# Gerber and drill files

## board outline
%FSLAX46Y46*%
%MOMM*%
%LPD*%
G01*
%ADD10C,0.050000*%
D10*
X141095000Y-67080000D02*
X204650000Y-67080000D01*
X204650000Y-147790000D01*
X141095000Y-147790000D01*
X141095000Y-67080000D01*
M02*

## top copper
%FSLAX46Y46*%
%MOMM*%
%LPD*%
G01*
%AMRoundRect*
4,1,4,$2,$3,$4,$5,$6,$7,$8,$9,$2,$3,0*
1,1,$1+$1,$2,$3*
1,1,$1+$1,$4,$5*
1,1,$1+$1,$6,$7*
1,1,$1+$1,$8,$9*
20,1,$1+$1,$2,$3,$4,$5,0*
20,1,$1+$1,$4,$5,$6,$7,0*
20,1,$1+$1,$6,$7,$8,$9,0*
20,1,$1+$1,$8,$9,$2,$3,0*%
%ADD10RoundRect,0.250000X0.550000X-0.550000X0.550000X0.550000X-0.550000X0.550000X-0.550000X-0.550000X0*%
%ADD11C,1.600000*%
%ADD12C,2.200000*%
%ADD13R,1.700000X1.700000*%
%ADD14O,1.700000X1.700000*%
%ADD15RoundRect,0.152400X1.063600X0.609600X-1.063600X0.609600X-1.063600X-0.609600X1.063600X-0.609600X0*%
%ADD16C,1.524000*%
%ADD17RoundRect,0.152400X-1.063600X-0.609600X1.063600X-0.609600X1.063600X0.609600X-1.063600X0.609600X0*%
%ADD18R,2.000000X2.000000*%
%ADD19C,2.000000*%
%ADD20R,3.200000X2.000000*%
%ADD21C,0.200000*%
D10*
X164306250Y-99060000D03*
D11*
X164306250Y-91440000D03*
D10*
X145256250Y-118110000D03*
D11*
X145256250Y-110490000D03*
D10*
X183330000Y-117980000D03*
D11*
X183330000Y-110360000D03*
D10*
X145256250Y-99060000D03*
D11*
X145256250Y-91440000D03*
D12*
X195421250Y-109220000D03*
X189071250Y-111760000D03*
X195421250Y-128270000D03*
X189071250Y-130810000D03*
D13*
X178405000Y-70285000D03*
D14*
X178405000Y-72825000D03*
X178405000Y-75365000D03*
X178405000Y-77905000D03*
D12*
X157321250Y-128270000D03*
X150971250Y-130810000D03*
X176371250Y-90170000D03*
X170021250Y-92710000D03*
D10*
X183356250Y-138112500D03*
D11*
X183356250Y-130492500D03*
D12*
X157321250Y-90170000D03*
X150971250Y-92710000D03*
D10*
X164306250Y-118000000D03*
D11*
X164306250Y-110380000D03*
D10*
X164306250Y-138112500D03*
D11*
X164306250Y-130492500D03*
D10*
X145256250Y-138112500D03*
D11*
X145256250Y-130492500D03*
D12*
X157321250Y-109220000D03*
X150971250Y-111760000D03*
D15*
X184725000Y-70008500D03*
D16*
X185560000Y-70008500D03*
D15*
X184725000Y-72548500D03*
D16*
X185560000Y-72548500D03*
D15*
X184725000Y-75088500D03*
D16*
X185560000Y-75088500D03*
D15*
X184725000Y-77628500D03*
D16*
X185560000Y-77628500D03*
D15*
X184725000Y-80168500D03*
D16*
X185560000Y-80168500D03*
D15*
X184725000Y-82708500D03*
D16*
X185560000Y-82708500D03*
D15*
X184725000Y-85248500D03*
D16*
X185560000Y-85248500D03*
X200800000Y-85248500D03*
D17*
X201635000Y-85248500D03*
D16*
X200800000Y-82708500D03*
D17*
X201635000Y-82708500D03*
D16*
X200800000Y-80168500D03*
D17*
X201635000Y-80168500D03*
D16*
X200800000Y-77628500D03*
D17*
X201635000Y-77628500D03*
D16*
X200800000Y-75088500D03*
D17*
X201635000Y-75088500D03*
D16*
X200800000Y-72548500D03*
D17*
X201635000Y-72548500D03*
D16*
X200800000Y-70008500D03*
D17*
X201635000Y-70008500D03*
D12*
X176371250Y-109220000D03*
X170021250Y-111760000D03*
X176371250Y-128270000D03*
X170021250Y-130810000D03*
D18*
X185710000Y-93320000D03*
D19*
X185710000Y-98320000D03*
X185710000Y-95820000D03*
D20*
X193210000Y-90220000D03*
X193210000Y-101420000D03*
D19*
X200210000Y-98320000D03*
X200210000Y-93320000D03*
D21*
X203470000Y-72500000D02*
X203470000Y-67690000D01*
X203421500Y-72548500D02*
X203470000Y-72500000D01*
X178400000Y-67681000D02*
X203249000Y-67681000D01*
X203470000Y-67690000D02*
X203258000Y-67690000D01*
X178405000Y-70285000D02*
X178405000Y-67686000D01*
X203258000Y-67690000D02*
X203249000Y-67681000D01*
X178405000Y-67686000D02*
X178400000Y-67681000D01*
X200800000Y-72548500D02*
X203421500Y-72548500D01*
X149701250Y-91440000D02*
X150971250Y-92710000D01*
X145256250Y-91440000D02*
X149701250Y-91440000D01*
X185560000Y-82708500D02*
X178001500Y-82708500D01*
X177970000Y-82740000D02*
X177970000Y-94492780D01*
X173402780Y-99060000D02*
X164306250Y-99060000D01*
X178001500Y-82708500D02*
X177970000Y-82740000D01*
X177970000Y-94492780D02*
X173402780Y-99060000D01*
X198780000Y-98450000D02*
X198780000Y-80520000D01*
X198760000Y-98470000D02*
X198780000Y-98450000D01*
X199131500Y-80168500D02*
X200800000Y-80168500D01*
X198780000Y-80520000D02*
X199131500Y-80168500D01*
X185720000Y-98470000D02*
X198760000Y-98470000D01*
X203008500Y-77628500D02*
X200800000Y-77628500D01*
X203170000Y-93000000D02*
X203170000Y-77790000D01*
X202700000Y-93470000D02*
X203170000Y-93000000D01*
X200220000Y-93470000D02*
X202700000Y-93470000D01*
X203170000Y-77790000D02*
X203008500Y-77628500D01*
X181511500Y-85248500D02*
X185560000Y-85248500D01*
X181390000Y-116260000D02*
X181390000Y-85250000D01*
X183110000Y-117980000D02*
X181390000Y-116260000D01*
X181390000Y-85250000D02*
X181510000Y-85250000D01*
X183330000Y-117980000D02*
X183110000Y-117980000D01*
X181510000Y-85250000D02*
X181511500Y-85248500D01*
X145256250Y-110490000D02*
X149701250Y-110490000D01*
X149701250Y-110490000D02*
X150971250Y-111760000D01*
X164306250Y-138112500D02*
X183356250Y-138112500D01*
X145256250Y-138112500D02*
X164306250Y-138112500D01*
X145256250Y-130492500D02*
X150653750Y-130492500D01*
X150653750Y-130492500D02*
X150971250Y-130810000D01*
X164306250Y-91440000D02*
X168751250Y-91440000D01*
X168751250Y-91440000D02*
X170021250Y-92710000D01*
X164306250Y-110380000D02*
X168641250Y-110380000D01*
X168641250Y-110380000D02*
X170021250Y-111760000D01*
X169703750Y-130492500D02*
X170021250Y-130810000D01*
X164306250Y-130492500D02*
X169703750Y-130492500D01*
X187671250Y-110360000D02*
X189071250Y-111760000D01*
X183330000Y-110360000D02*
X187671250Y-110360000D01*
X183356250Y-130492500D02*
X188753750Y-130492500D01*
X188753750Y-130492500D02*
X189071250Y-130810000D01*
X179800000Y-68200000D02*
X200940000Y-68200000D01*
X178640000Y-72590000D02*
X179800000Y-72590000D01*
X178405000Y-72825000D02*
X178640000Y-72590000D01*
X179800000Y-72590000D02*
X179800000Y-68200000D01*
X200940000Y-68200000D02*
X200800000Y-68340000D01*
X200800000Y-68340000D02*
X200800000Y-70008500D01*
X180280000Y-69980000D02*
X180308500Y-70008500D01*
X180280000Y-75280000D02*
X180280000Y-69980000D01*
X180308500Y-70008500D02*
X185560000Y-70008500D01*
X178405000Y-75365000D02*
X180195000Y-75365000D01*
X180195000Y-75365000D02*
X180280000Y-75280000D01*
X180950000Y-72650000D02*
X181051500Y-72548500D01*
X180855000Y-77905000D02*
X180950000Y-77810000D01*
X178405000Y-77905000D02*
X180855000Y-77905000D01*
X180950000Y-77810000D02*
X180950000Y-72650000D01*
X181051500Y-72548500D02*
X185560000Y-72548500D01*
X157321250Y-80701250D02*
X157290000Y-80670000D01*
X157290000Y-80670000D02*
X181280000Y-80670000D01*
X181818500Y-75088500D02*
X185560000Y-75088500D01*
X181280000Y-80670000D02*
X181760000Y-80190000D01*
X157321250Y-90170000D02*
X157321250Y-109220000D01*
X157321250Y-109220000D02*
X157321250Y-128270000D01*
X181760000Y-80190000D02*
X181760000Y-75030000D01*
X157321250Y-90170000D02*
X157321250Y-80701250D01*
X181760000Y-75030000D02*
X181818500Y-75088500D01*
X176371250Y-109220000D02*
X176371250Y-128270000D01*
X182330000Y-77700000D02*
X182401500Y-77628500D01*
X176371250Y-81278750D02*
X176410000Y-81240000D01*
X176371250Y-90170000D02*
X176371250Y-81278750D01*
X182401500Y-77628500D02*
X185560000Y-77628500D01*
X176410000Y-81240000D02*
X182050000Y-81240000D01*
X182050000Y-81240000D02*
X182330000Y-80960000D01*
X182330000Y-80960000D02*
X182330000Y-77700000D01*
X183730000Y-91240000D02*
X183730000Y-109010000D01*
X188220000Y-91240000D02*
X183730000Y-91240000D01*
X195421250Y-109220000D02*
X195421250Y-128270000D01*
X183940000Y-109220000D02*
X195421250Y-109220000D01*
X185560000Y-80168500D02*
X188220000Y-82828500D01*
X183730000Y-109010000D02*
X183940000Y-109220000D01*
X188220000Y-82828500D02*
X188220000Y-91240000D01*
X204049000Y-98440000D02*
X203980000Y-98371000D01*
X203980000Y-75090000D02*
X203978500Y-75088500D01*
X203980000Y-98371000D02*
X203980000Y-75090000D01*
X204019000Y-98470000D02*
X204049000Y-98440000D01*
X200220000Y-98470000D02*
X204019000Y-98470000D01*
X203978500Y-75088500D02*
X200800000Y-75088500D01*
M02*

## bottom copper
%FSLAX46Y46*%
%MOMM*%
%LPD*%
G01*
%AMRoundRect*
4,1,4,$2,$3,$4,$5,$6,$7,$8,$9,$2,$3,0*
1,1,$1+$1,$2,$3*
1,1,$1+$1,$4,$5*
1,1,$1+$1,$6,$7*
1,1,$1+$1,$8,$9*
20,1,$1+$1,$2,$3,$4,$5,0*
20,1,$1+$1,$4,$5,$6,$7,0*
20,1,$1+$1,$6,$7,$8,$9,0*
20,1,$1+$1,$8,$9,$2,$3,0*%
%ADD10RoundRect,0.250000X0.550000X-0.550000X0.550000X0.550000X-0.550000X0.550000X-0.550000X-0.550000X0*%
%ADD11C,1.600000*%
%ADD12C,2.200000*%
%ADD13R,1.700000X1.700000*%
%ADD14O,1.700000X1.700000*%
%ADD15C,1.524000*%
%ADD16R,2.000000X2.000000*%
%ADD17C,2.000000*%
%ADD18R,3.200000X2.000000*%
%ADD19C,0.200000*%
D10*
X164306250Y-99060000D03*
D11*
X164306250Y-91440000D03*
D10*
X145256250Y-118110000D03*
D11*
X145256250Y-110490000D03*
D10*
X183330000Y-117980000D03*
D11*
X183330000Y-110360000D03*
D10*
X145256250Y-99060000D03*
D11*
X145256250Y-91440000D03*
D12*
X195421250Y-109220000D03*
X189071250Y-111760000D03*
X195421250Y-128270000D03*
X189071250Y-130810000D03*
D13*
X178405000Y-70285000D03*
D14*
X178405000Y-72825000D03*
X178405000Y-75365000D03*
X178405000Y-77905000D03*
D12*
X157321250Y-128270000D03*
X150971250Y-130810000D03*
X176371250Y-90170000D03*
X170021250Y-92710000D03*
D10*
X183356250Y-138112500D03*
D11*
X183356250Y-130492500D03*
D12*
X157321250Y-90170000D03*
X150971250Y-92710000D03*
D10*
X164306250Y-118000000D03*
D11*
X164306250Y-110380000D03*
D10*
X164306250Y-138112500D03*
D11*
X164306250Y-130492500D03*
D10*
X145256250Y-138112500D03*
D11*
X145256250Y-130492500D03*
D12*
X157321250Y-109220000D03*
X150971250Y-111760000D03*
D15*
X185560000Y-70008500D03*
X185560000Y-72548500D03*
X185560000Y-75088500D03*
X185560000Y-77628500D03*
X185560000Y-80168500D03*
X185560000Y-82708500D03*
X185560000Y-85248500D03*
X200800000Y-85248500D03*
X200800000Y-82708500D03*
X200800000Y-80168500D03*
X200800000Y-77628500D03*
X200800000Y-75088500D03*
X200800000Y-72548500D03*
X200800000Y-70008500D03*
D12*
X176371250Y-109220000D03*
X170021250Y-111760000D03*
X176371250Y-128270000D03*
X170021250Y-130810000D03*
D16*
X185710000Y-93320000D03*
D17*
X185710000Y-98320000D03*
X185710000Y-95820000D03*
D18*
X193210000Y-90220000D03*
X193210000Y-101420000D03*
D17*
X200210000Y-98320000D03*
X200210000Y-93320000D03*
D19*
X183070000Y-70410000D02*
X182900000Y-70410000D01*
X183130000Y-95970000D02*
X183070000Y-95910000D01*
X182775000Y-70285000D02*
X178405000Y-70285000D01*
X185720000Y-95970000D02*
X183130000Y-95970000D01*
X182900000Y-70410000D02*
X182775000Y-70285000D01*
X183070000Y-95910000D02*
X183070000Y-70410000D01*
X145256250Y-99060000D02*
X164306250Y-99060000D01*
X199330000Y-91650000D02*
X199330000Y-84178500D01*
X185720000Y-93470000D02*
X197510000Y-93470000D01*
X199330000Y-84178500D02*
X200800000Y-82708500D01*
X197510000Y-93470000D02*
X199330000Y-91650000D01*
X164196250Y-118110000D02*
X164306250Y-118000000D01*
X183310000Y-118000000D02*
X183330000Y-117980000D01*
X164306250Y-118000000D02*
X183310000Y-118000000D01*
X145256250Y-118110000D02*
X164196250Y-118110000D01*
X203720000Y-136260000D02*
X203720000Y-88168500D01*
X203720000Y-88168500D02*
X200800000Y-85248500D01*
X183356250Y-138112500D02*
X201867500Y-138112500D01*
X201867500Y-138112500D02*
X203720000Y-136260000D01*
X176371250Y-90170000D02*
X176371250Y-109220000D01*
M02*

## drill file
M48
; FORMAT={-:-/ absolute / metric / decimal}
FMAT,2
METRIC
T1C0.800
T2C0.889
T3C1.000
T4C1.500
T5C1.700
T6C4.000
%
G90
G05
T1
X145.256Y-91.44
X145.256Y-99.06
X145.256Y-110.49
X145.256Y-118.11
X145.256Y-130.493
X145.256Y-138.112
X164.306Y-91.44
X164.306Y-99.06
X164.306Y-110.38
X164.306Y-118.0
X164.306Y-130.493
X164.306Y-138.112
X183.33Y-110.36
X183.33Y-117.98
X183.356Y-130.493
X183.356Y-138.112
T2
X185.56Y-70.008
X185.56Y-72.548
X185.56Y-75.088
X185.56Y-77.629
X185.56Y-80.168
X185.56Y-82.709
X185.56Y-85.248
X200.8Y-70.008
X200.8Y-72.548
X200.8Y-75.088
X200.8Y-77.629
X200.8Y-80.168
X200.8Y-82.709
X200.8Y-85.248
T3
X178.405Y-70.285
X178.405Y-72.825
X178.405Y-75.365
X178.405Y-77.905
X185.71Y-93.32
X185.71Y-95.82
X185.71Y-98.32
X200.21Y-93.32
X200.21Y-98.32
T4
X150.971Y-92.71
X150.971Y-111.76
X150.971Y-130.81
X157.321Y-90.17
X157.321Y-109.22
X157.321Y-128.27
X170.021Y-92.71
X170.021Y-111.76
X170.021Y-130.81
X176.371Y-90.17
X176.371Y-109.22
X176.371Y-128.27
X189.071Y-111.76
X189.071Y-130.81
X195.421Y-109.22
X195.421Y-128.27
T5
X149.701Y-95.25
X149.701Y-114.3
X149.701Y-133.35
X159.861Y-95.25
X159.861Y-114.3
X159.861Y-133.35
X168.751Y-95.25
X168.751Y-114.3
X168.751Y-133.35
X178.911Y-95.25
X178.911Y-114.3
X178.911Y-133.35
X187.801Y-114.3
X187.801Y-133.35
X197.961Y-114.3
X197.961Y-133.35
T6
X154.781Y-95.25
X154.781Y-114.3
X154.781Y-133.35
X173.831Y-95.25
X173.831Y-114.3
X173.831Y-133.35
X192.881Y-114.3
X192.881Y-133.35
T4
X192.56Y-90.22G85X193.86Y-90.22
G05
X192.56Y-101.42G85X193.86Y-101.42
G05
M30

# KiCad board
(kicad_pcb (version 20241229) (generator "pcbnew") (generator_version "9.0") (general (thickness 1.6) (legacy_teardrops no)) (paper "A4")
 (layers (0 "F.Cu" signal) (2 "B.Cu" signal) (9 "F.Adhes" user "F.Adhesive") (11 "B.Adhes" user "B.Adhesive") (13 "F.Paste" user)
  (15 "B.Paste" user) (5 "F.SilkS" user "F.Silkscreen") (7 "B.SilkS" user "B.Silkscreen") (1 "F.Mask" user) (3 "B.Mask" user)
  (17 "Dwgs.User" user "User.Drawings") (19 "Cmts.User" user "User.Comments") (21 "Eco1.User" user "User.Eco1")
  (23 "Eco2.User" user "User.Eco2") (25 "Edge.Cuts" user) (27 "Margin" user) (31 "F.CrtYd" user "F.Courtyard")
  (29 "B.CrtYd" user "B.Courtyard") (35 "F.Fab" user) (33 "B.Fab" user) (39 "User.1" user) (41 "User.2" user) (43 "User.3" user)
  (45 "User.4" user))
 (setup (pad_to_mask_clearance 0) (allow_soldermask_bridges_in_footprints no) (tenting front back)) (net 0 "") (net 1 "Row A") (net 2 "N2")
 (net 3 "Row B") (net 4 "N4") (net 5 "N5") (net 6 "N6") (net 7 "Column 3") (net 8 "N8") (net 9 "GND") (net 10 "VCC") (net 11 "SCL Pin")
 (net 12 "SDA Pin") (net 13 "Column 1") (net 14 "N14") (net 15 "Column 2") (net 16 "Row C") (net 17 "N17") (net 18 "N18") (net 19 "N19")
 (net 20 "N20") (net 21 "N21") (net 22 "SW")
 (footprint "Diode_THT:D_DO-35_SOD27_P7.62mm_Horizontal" (layer "F.Cu") (at 164.30625 99.06 90)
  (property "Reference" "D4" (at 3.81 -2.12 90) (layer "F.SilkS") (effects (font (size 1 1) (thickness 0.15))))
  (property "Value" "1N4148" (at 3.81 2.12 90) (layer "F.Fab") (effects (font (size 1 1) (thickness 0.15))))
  (pad "1" thru_hole roundrect (at 0 0 90) (size 1.6 1.6) (drill 0.8) (layers "*.Cu" "*.Mask") (remove_unused_layers no)
   (roundrect_rratio 0.15625) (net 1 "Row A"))
  (pad "2" thru_hole circle (at 7.62 0 90) (size 1.6 1.6) (drill 0.8) (layers "*.Cu" "*.Mask") (remove_unused_layers no) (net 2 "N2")))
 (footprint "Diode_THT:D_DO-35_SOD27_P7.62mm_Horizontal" (layer "F.Cu") (at 145.25625 118.11 90)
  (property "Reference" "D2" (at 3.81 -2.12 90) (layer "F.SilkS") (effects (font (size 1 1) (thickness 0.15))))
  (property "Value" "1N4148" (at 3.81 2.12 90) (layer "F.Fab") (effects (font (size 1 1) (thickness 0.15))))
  (pad "1" thru_hole roundrect (at 0 0 90) (size 1.6 1.6) (drill 0.8) (layers "*.Cu" "*.Mask") (remove_unused_layers no)
   (roundrect_rratio 0.15625) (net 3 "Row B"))
  (pad "2" thru_hole circle (at 7.62 0 90) (size 1.6 1.6) (drill 0.8) (layers "*.Cu" "*.Mask") (remove_unused_layers no) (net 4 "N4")))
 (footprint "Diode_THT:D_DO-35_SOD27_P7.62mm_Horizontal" (layer "F.Cu") (at 183.33 117.98 90)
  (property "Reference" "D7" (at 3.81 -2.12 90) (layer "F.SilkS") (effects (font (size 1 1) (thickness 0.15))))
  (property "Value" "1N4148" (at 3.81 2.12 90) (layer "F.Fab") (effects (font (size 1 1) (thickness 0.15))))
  (pad "1" thru_hole roundrect (at 0 0 90) (size 1.6 1.6) (drill 0.8) (layers "*.Cu" "*.Mask") (remove_unused_layers no)
   (roundrect_rratio 0.15625) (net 3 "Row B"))
  (pad "2" thru_hole circle (at 7.62 0 90) (size 1.6 1.6) (drill 0.8) (layers "*.Cu" "*.Mask") (remove_unused_layers no) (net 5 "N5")))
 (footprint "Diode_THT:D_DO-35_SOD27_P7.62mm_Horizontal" (layer "F.Cu") (at 145.25625 99.06 90)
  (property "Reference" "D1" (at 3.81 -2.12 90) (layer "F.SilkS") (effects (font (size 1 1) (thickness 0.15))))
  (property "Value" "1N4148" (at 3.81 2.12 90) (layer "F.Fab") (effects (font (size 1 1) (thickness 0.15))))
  (pad "1" thru_hole roundrect (at 0 0 90) (size 1.6 1.6) (drill 0.8) (layers "*.Cu" "*.Mask") (remove_unused_layers no)
   (roundrect_rratio 0.15625) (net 1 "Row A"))
  (pad "2" thru_hole circle (at 7.62 0 90) (size 1.6 1.6) (drill 0.8) (layers "*.Cu" "*.Mask") (remove_unused_layers no) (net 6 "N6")))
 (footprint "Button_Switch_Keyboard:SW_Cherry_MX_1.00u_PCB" (layer "F.Cu") (at 195.42125 109.22)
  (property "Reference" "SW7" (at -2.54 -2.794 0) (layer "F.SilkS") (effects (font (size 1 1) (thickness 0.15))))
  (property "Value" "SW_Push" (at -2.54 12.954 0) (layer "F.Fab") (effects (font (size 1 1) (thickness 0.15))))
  (pad "" np_thru_hole circle (at -7.62 5.08) (size 1.7 1.7) (drill 1.7) (layers "*.Cu" "*.Mask"))
  (pad "" np_thru_hole circle (at -2.54 5.08) (size 4 4) (drill 4) (layers "*.Cu" "*.Mask"))
  (pad "" np_thru_hole circle (at 2.54 5.08) (size 1.7 1.7) (drill 1.7) (layers "*.Cu" "*.Mask"))
  (pad "1" thru_hole circle (at 0 0) (size 2.2 2.2) (drill 1.5) (layers "*.Cu" "*.Mask") (remove_unused_layers no) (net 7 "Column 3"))
  (pad "2" thru_hole circle (at -6.35 2.54) (size 2.2 2.2) (drill 1.5) (layers "*.Cu" "*.Mask") (remove_unused_layers no) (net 5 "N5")))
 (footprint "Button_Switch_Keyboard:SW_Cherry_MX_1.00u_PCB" (layer "F.Cu") (at 195.42125 128.27)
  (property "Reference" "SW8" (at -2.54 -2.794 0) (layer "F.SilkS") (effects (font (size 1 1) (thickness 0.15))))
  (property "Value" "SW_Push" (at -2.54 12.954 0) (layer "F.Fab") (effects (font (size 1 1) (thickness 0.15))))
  (pad "" np_thru_hole circle (at -7.62 5.08) (size 1.7 1.7) (drill 1.7) (layers "*.Cu" "*.Mask"))
  (pad "" np_thru_hole circle (at -2.54 5.08) (size 4 4) (drill 4) (layers "*.Cu" "*.Mask"))
  (pad "" np_thru_hole circle (at 2.54 5.08) (size 1.7 1.7) (drill 1.7) (layers "*.Cu" "*.Mask"))
  (pad "1" thru_hole circle (at 0 0) (size 2.2 2.2) (drill 1.5) (layers "*.Cu" "*.Mask") (remove_unused_layers no) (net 7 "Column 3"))
  (pad "2" thru_hole circle (at -6.35 2.54) (size 2.2 2.2) (drill 1.5) (layers "*.Cu" "*.Mask") (remove_unused_layers no) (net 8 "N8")))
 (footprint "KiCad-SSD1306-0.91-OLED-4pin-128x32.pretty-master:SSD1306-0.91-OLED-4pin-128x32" (layer "F.Cu") (at 141.905 68.095)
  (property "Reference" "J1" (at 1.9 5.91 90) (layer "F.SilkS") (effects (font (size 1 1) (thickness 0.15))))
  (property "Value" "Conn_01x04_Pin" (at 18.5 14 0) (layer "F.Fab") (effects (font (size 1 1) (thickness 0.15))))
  (pad "1" thru_hole rect (at 36.5 2.19) (size 1.7 1.7) (drill 1) (layers "*.Cu" "*.Mask") (remove_unused_layers no) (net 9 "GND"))
  (pad "2" thru_hole oval (at 36.5 4.73) (size 1.7 1.7) (drill 1) (layers "*.Cu" "*.Mask") (remove_unused_layers no) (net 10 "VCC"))
  (pad "3" thru_hole oval (at 36.5 7.27) (size 1.7 1.7) (drill 1) (layers "*.Cu" "*.Mask") (remove_unused_layers no) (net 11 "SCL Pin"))
  (pad "4" thru_hole oval (at 36.5 9.81) (size 1.7 1.7) (drill 1) (layers "*.Cu" "*.Mask") (remove_unused_layers no) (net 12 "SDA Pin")))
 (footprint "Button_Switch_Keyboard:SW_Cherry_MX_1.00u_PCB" (layer "F.Cu") (at 157.32125 128.27)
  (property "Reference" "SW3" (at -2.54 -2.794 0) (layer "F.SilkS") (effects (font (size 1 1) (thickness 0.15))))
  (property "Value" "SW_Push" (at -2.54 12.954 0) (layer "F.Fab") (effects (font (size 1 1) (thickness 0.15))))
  (pad "" np_thru_hole circle (at -7.62 5.08) (size 1.7 1.7) (drill 1.7) (layers "*.Cu" "*.Mask"))
  (pad "" np_thru_hole circle (at -2.54 5.08) (size 4 4) (drill 4) (layers "*.Cu" "*.Mask"))
  (pad "" np_thru_hole circle (at 2.54 5.08) (size 1.7 1.7) (drill 1.7) (layers "*.Cu" "*.Mask"))
  (pad "1" thru_hole circle (at 0 0) (size 2.2 2.2) (drill 1.5) (layers "*.Cu" "*.Mask") (remove_unused_layers no) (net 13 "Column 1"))
  (pad "2" thru_hole circle (at -6.35 2.54) (size 2.2 2.2) (drill 1.5) (layers "*.Cu" "*.Mask") (remove_unused_layers no) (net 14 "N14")))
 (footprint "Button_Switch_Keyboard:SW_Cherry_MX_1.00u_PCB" (layer "F.Cu") (at 176.37125 90.17)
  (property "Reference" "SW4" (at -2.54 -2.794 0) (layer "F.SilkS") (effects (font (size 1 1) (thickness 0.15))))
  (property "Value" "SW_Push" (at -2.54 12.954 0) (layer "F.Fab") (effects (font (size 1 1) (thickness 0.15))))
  (pad "" np_thru_hole circle (at -7.62 5.08) (size 1.7 1.7) (drill 1.7) (layers "*.Cu" "*.Mask"))
  (pad "" np_thru_hole circle (at -2.54 5.08) (size 4 4) (drill 4) (layers "*.Cu" "*.Mask"))
  (pad "" np_thru_hole circle (at 2.54 5.08) (size 1.7 1.7) (drill 1.7) (layers "*.Cu" "*.Mask"))
  (pad "1" thru_hole circle (at 0 0) (size 2.2 2.2) (drill 1.5) (layers "*.Cu" "*.Mask") (remove_unused_layers no) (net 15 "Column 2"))
  (pad "2" thru_hole circle (at -6.35 2.54) (size 2.2 2.2) (drill 1.5) (layers "*.Cu" "*.Mask") (remove_unused_layers no) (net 2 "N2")))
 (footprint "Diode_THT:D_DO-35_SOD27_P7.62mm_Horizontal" (layer "F.Cu") (at 183.35625 138.1125 90)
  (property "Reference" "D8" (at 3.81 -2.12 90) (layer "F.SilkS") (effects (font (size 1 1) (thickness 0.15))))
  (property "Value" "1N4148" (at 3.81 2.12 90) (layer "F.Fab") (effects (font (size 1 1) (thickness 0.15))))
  (pad "1" thru_hole roundrect (at 0 0 90) (size 1.6 1.6) (drill 0.8) (layers "*.Cu" "*.Mask") (remove_unused_layers no)
   (roundrect_rratio 0.15625) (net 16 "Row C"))
  (pad "2" thru_hole circle (at 7.62 0 90) (size 1.6 1.6) (drill 0.8) (layers "*.Cu" "*.Mask") (remove_unused_layers no) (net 8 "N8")))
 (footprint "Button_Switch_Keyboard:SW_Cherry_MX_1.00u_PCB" (layer "F.Cu") (at 157.32125 90.17)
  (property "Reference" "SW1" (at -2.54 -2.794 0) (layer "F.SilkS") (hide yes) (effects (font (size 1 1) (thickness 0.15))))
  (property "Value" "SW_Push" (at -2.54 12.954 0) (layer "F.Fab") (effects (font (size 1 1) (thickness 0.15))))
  (pad "" np_thru_hole circle (at -7.62 5.08) (size 1.7 1.7) (drill 1.7) (layers "*.Cu" "*.Mask"))
  (pad "" np_thru_hole circle (at -2.54 5.08) (size 4 4) (drill 4) (layers "*.Cu" "*.Mask"))
  (pad "" np_thru_hole circle (at 2.54 5.08) (size 1.7 1.7) (drill 1.7) (layers "*.Cu" "*.Mask"))
  (pad "1" thru_hole circle (at 0 0) (size 2.2 2.2) (drill 1.5) (layers "*.Cu" "*.Mask") (remove_unused_layers no) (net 13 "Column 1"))
  (pad "2" thru_hole circle (at -6.35 2.54) (size 2.2 2.2) (drill 1.5) (layers "*.Cu" "*.Mask") (remove_unused_layers no) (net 6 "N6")))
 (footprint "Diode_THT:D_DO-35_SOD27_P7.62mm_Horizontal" (layer "F.Cu") (at 164.30625 118 90)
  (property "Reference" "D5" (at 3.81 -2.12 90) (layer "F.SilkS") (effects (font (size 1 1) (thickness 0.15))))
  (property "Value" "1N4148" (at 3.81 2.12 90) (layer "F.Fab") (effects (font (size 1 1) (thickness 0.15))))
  (pad "1" thru_hole roundrect (at 0 0 90) (size 1.6 1.6) (drill 0.8) (layers "*.Cu" "*.Mask") (remove_unused_layers no)
   (roundrect_rratio 0.15625) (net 3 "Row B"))
  (pad "2" thru_hole circle (at 7.62 0 90) (size 1.6 1.6) (drill 0.8) (layers "*.Cu" "*.Mask") (remove_unused_layers no) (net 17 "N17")))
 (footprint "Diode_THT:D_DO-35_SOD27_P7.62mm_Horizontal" (layer "F.Cu") (at 164.30625 138.1125 90)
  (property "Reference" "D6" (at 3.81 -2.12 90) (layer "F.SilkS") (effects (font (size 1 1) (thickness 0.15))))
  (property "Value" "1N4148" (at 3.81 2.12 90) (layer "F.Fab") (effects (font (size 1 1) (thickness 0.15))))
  (pad "1" thru_hole roundrect (at 0 0 90) (size 1.6 1.6) (drill 0.8) (layers "*.Cu" "*.Mask") (remove_unused_layers no)
   (roundrect_rratio 0.15625) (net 16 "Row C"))
  (pad "2" thru_hole circle (at 7.62 0 90) (size 1.6 1.6) (drill 0.8) (layers "*.Cu" "*.Mask") (remove_unused_layers no) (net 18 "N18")))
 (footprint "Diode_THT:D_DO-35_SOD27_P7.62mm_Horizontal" (layer "F.Cu") (at 145.25625 138.1125 90)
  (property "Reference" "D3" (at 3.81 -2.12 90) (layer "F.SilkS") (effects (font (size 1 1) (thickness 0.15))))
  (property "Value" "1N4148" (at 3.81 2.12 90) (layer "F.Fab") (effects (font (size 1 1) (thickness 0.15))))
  (pad "1" thru_hole roundrect (at 0 0 90) (size 1.6 1.6) (drill 0.8) (layers "*.Cu" "*.Mask") (remove_unused_layers no)
   (roundrect_rratio 0.15625) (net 16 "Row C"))
  (pad "2" thru_hole circle (at 7.62 0 90) (size 1.6 1.6) (drill 0.8) (layers "*.Cu" "*.Mask") (remove_unused_layers no) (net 14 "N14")))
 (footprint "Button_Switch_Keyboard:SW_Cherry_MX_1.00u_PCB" (layer "F.Cu") (at 157.32125 109.22)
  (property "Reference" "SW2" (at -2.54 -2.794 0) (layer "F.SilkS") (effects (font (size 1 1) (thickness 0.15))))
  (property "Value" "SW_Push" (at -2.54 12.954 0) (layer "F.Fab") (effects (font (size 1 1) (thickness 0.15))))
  (pad "" np_thru_hole circle (at -7.62 5.08) (size 1.7 1.7) (drill 1.7) (layers "*.Cu" "*.Mask"))
  (pad "" np_thru_hole circle (at -2.54 5.08) (size 4 4) (drill 4) (layers "*.Cu" "*.Mask"))
  (pad "" np_thru_hole circle (at 2.54 5.08) (size 1.7 1.7) (drill 1.7) (layers "*.Cu" "*.Mask"))
  (pad "1" thru_hole circle (at 0 0) (size 2.2 2.2) (drill 1.5) (layers "*.Cu" "*.Mask") (remove_unused_layers no) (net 13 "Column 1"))
  (pad "2" thru_hole circle (at -6.35 2.54) (size 2.2 2.2) (drill 1.5) (layers "*.Cu" "*.Mask") (remove_unused_layers no) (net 4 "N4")))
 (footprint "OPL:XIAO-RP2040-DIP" (layer "F.Cu") (at 193.18 77.6285)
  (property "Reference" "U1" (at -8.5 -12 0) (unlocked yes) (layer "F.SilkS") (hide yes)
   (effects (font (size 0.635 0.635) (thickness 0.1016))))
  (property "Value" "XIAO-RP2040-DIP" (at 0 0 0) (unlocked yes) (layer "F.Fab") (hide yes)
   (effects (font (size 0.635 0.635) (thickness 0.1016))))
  (pad "1" smd roundrect (at -8.455 -7.62 180) (size 2.432 1.524) (layers "F.Cu" "F.Mask") (roundrect_rratio 0.1) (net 11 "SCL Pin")
   (thermal_bridge_angle 45))
  (pad "1" thru_hole circle (at -7.62 -7.62 180) (size 1.524 1.524) (drill 0.889) (layers "*.Cu" "*.Mask") (remove_unused_layers no)
   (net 11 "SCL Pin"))
  (pad "2" smd roundrect (at -8.455 -5.08 180) (size 2.432 1.524) (layers "F.Cu" "F.Mask") (roundrect_rratio 0.1) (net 12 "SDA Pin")
   (thermal_bridge_angle 45))
  (pad "2" thru_hole circle (at -7.62 -5.08 180) (size 1.524 1.524) (drill 0.889) (layers "*.Cu" "*.Mask") (remove_unused_layers no)
   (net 12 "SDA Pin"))
  (pad "3" smd roundrect (at -8.455 -2.54 180) (size 2.432 1.524) (layers "F.Cu" "F.Mask") (roundrect_rratio 0.1) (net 13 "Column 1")
   (thermal_bridge_angle 45))
  (pad "3" thru_hole circle (at -7.62 -2.54 180) (size 1.524 1.524) (drill 0.889) (layers "*.Cu" "*.Mask") (remove_unused_layers no)
   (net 13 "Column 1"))
  (pad "4" smd roundrect (at -8.455 0 180) (size 2.432 1.524) (layers "F.Cu" "F.Mask") (roundrect_rratio 0.1) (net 15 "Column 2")
   (thermal_bridge_angle 45))
  (pad "4" thru_hole circle (at -7.62 0 180) (size 1.524 1.524) (drill 0.889) (layers "*.Cu" "*.Mask") (remove_unused_layers no)
   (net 15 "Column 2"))
  (pad "5" smd roundrect (at -8.455 2.54 180) (size 2.432 1.524) (layers "F.Cu" "F.Mask") (roundrect_rratio 0.1) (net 7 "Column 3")
   (thermal_bridge_angle 45))
  (pad "5" thru_hole circle (at -7.62 2.54 180) (size 1.524 1.524) (drill 0.889) (layers "*.Cu" "*.Mask") (remove_unused_layers no)
   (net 7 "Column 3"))
  (pad "6" smd roundrect (at -8.455 5.08 180) (size 2.432 1.524) (layers "F.Cu" "F.Mask") (roundrect_rratio 0.1) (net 1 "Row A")
   (thermal_bridge_angle 45))
  (pad "6" thru_hole circle (at -7.62 5.08 180) (size 1.524 1.524) (drill 0.889) (layers "*.Cu" "*.Mask") (remove_unused_layers no)
   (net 1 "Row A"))
  (pad "7" smd roundrect (at -8.455 7.62 180) (size 2.432 1.524) (layers "F.Cu" "F.Mask") (roundrect_rratio 0.1) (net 3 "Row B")
   (thermal_bridge_angle 45))
  (pad "7" thru_hole circle (at -7.62 7.62 180) (size 1.524 1.524) (drill 0.889) (layers "*.Cu" "*.Mask") (remove_unused_layers no)
   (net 3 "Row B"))
  (pad "8" thru_hole circle (at 7.62 7.62) (size 1.524 1.524) (drill 0.889) (layers "*.Cu" "*.Mask") (remove_unused_layers no)
   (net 16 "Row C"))
  (pad "8" smd roundrect (at 8.455 7.62) (size 2.432 1.524) (layers "F.Cu" "F.Mask") (roundrect_rratio 0.1) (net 16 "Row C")
   (thermal_bridge_angle 45))
  (pad "9" thru_hole circle (at 7.62 5.08) (size 1.524 1.524) (drill 0.889) (layers "*.Cu" "*.Mask") (remove_unused_layers no)
   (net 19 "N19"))
  (pad "9" smd roundrect (at 8.455 5.08) (size 2.432 1.524) (layers "F.Cu" "F.Mask") (roundrect_rratio 0.1) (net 19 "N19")
   (thermal_bridge_angle 45))
  (pad "10" thru_hole circle (at 7.62 2.54) (size 1.524 1.524) (drill 0.889) (layers "*.Cu" "*.Mask") (remove_unused_layers no)
   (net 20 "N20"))
  (pad "10" smd roundrect (at 8.455 2.54) (size 2.432 1.524) (layers "F.Cu" "F.Mask") (roundrect_rratio 0.1) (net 20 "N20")
   (thermal_bridge_angle 45))
  (pad "11" thru_hole circle (at 7.62 0) (size 1.524 1.524) (drill 0.889) (layers "*.Cu" "*.Mask") (remove_unused_layers no) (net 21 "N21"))
  (pad "11" smd roundrect (at 8.455 0) (size 2.432 1.524) (layers "F.Cu" "F.Mask") (roundrect_rratio 0.1) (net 21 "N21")
   (thermal_bridge_angle 45))
  (pad "12" thru_hole circle (at 7.62 -2.54) (size 1.524 1.524) (drill 0.889) (layers "*.Cu" "*.Mask") (remove_unused_layers no)
   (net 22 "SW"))
  (pad "12" smd roundrect (at 8.455 -2.54) (size 2.432 1.524) (layers "F.Cu" "F.Mask") (roundrect_rratio 0.1) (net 22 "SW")
   (thermal_bridge_angle 45))
  (pad "13" thru_hole circle (at 7.62 -5.08) (size 1.524 1.524) (drill 0.889) (layers "*.Cu" "*.Mask") (remove_unused_layers no)
   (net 9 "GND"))
  (pad "13" smd roundrect (at 8.455 -5.08) (size 2.432 1.524) (layers "F.Cu" "F.Mask") (roundrect_rratio 0.1) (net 9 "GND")
   (thermal_bridge_angle 45))
  (pad "14" thru_hole circle (at 7.62 -7.62) (size 1.524 1.524) (drill 0.889) (layers "*.Cu" "*.Mask") (remove_unused_layers no)
   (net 10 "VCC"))
  (pad "14" smd roundrect (at 8.455 -7.62) (size 2.432 1.524) (layers "F.Cu" "F.Mask") (roundrect_rratio 0.1) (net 10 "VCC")
   (thermal_bridge_angle 45)))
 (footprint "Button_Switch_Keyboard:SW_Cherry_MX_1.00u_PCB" (layer "F.Cu") (at 176.37125 109.22)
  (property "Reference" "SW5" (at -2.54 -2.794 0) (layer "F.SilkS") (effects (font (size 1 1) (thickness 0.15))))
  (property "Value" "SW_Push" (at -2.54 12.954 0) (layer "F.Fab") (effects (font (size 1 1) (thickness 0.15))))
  (pad "" np_thru_hole circle (at -7.62 5.08) (size 1.7 1.7) (drill 1.7) (layers "*.Cu" "*.Mask"))
  (pad "" np_thru_hole circle (at -2.54 5.08) (size 4 4) (drill 4) (layers "*.Cu" "*.Mask"))
  (pad "" np_thru_hole circle (at 2.54 5.08) (size 1.7 1.7) (drill 1.7) (layers "*.Cu" "*.Mask"))
  (pad "1" thru_hole circle (at 0 0) (size 2.2 2.2) (drill 1.5) (layers "*.Cu" "*.Mask") (remove_unused_layers no) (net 15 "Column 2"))
  (pad "2" thru_hole circle (at -6.35 2.54) (size 2.2 2.2) (drill 1.5) (layers "*.Cu" "*.Mask") (remove_unused_layers no) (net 17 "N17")))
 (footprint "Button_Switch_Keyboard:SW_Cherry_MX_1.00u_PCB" (layer "F.Cu") (at 176.37125 128.27)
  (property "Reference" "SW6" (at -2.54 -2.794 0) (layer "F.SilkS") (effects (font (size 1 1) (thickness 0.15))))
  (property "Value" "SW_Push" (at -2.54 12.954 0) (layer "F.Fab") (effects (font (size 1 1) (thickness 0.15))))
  (pad "" np_thru_hole circle (at -7.62 5.08) (size 1.7 1.7) (drill 1.7) (layers "*.Cu" "*.Mask"))
  (pad "" np_thru_hole circle (at -2.54 5.08) (size 4 4) (drill 4) (layers "*.Cu" "*.Mask"))
  (pad "" np_thru_hole circle (at 2.54 5.08) (size 1.7 1.7) (drill 1.7) (layers "*.Cu" "*.Mask"))
  (pad "1" thru_hole circle (at 0 0) (size 2.2 2.2) (drill 1.5) (layers "*.Cu" "*.Mask") (remove_unused_layers no) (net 15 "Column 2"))
  (pad "2" thru_hole circle (at -6.35 2.54) (size 2.2 2.2) (drill 1.5) (layers "*.Cu" "*.Mask") (remove_unused_layers no) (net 18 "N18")))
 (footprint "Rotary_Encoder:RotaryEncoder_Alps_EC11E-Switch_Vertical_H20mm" (layer "F.Cu") (at 185.71 93.32)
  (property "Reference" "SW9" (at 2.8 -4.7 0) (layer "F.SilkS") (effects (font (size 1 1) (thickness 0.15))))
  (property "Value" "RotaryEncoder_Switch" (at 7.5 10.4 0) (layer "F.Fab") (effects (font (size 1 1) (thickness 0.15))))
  (pad "A" thru_hole rect (at 0 0) (size 2 2) (drill 1) (layers "*.Cu" "*.Mask") (remove_unused_layers no) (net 19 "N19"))
  (pad "B" thru_hole circle (at 0 5) (size 2 2) (drill 1) (layers "*.Cu" "*.Mask") (remove_unused_layers no) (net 20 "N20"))
  (pad "C" thru_hole circle (at 0 2.5) (size 2 2) (drill 1) (layers "*.Cu" "*.Mask") (remove_unused_layers no) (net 9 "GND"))
  (pad "MP" thru_hole rect (at 7.5 -3.1) (size 3.2 2) (drill oval 2.8 1.5) (layers "*.Cu" "*.Mask") (remove_unused_layers no))
  (pad "MP" thru_hole rect (at 7.5 8.1) (size 3.2 2) (drill oval 2.8 1.5) (layers "*.Cu" "*.Mask") (remove_unused_layers no))
  (pad "S1" thru_hole circle (at 14.5 5) (size 2 2) (drill 1) (layers "*.Cu" "*.Mask") (remove_unused_layers no) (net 22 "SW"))
  (pad "S2" thru_hole circle (at 14.5 0) (size 2 2) (drill 1) (layers "*.Cu" "*.Mask") (remove_unused_layers no) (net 21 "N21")))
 (gr_rect (start 141.095 67.08) (end 204.65 147.79) (stroke (width 0.05) (type default)) (fill no) (layer "Edge.Cuts"))
 (segment (start 203.47 72.5) (end 203.47 67.69) (width 0.2) (layer "F.Cu") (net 9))
 (segment (start 203.4215 72.5485) (end 203.47 72.5) (width 0.2) (layer "F.Cu") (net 9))
 (segment (start 178.4 67.681) (end 203.249 67.681) (width 0.2) (layer "F.Cu") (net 9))
 (segment (start 203.47 67.69) (end 203.258 67.69) (width 0.2) (layer "F.Cu") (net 9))
 (segment (start 178.405 70.285) (end 178.405 67.686) (width 0.2) (layer "F.Cu") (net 9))
 (segment (start 203.258 67.69) (end 203.249 67.681) (width 0.2) (layer "F.Cu") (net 9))
 (segment (start 178.405 67.686) (end 178.4 67.681) (width 0.2) (layer "F.Cu") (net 9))
 (segment (start 200.8 72.5485) (end 203.4215 72.5485) (width 0.2) (layer "F.Cu") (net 9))
 (segment (start 183.07 70.41) (end 182.9 70.41) (width 0.2) (layer "B.Cu") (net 9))
 (segment (start 183.13 95.97) (end 183.07 95.91) (width 0.2) (layer "B.Cu") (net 9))
 (segment (start 182.775 70.285) (end 178.405 70.285) (width 0.2) (layer "B.Cu") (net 9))
 (segment (start 185.72 95.97) (end 183.13 95.97) (width 0.2) (layer "B.Cu") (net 9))
 (segment (start 182.9 70.41) (end 182.775 70.285) (width 0.2) (layer "B.Cu") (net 9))
 (segment (start 183.07 95.91) (end 183.07 70.41) (width 0.2) (layer "B.Cu") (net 9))
 (segment (start 149.70125 91.44) (end 150.97125 92.71) (width 0.2) (layer "F.Cu") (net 6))
 (segment (start 145.25625 91.44) (end 149.70125 91.44) (width 0.2) (layer "F.Cu") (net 6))
 (segment (start 185.56 82.7085) (end 178.0015 82.7085) (width 0.2) (layer "F.Cu") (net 1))
 (segment (start 177.97 82.74) (end 177.97 94.49278) (width 0.2) (layer "F.Cu") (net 1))
 (segment (start 173.40278 99.06) (end 164.30625 99.06) (width 0.2) (layer "F.Cu") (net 1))
 (segment (start 178.0015 82.7085) (end 177.97 82.74) (width 0.2) (layer "F.Cu") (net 1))
 (segment (start 177.97 94.49278) (end 173.40278 99.06) (width 0.2) (layer "F.Cu") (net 1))
 (segment (start 145.25625 99.06) (end 164.30625 99.06) (width 0.2) (layer "B.Cu") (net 1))
 (segment (start 199.33 91.65) (end 199.33 84.1785) (width 0.2) (layer "B.Cu") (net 19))
 (segment (start 185.72 93.47) (end 197.51 93.47) (width 0.2) (layer "B.Cu") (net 19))
 (segment (start 199.33 84.1785) (end 200.8 82.7085) (width 0.2) (layer "B.Cu") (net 19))
 (segment (start 197.51 93.47) (end 199.33 91.65) (width 0.2) (layer "B.Cu") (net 19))
 (segment (start 198.78 98.45) (end 198.78 80.52) (width 0.2) (layer "F.Cu") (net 20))
 (segment (start 198.76 98.47) (end 198.78 98.45) (width 0.2) (layer "F.Cu") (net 20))
 (segment (start 199.1315 80.1685) (end 200.8 80.1685) (width 0.2) (layer "F.Cu") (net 20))
 (segment (start 198.78 80.52) (end 199.1315 80.1685) (width 0.2) (layer "F.Cu") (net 20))
 (segment (start 185.72 98.47) (end 198.76 98.47) (width 0.2) (layer "F.Cu") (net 20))
 (segment (start 203.0085 77.6285) (end 200.8 77.6285) (width 0.2) (layer "F.Cu") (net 21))
 (segment (start 203.17 93) (end 203.17 77.79) (width 0.2) (layer "F.Cu") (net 21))
 (segment (start 202.7 93.47) (end 203.17 93) (width 0.2) (layer "F.Cu") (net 21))
 (segment (start 200.22 93.47) (end 202.7 93.47) (width 0.2) (layer "F.Cu") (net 21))
 (segment (start 203.17 77.79) (end 203.0085 77.6285) (width 0.2) (layer "F.Cu") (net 21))
 (segment (start 181.5115 85.2485) (end 185.56 85.2485) (width 0.2) (layer "F.Cu") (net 3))
 (segment (start 181.39 116.26) (end 181.39 85.25) (width 0.2) (layer "F.Cu") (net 3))
 (segment (start 183.11 117.98) (end 181.39 116.26) (width 0.2) (layer "F.Cu") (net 3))
 (segment (start 181.39 85.25) (end 181.51 85.25) (width 0.2) (layer "F.Cu") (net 3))
 (segment (start 183.33 117.98) (end 183.11 117.98) (width 0.2) (layer "F.Cu") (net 3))
 (segment (start 181.51 85.25) (end 181.5115 85.2485) (width 0.2) (layer "F.Cu") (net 3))
 (segment (start 164.19625 118.11) (end 164.30625 118) (width 0.2) (layer "B.Cu") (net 3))
 (segment (start 183.31 118) (end 183.33 117.98) (width 0.2) (layer "B.Cu") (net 3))
 (segment (start 164.30625 118) (end 183.31 118) (width 0.2) (layer "B.Cu") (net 3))
 (segment (start 145.25625 118.11) (end 164.19625 118.11) (width 0.2) (layer "B.Cu") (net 3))
 (segment (start 145.25625 110.49) (end 149.70125 110.49) (width 0.2) (layer "F.Cu") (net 4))
 (segment (start 149.70125 110.49) (end 150.97125 111.76) (width 0.2) (layer "F.Cu") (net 4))
 (segment (start 164.30625 138.1125) (end 183.35625 138.1125) (width 0.2) (layer "F.Cu") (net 16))
 (segment (start 145.25625 138.1125) (end 164.30625 138.1125) (width 0.2) (layer "F.Cu") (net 16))
 (segment (start 203.72 136.26) (end 203.72 88.1685) (width 0.2) (layer "B.Cu") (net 16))
 (segment (start 203.72 88.1685) (end 200.8 85.2485) (width 0.2) (layer "B.Cu") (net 16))
 (segment (start 183.35625 138.1125) (end 201.8675 138.1125) (width 0.2) (layer "B.Cu") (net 16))
 (segment (start 201.8675 138.1125) (end 203.72 136.26) (width 0.2) (layer "B.Cu") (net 16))
 (segment (start 145.25625 130.4925) (end 150.65375 130.4925) (width 0.2) (layer "F.Cu") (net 14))
 (segment (start 150.65375 130.4925) (end 150.97125 130.81) (width 0.2) (layer "F.Cu") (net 14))
 (segment (start 164.30625 91.44) (end 168.75125 91.44) (width 0.2) (layer "F.Cu") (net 2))
 (segment (start 168.75125 91.44) (end 170.02125 92.71) (width 0.2) (layer "F.Cu") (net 2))
 (segment (start 164.30625 110.38) (end 168.64125 110.38) (width 0.2) (layer "F.Cu") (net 17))
 (segment (start 168.64125 110.38) (end 170.02125 111.76) (width 0.2) (layer "F.Cu") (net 17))
 (segment (start 169.70375 130.4925) (end 170.02125 130.81) (width 0.2) (layer "F.Cu") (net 18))
 (segment (start 164.30625 130.4925) (end 169.70375 130.4925) (width 0.2) (layer "F.Cu") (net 18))
 (segment (start 187.67125 110.36) (end 189.07125 111.76) (width 0.2) (layer "F.Cu") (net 5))
 (segment (start 183.33 110.36) (end 187.67125 110.36) (width 0.2) (layer "F.Cu") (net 5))
 (segment (start 183.35625 130.4925) (end 188.75375 130.4925) (width 0.2) (layer "F.Cu") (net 8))
 (segment (start 188.75375 130.4925) (end 189.07125 130.81) (width 0.2) (layer "F.Cu") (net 8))
 (segment (start 179.8 68.2) (end 200.94 68.2) (width 0.2) (layer "F.Cu") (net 10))
 (segment (start 178.64 72.59) (end 179.8 72.59) (width 0.2) (layer "F.Cu") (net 10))
 (segment (start 178.405 72.825) (end 178.64 72.59) (width 0.2) (layer "F.Cu") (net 10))
 (segment (start 179.8 72.59) (end 179.8 68.2) (width 0.2) (layer "F.Cu") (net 10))
 (segment (start 200.94 68.2) (end 200.8 68.34) (width 0.2) (layer "F.Cu") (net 10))
 (segment (start 200.8 68.34) (end 200.8 70.0085) (width 0.2) (layer "F.Cu") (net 10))
 (segment (start 180.28 69.98) (end 180.3085 70.0085) (width 0.2) (layer "F.Cu") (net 11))
 (segment (start 180.28 75.28) (end 180.28 69.98) (width 0.2) (layer "F.Cu") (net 11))
 (segment (start 180.3085 70.0085) (end 185.56 70.0085) (width 0.2) (layer "F.Cu") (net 11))
 (segment (start 178.405 75.365) (end 180.195 75.365) (width 0.2) (layer "F.Cu") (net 11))
 (segment (start 180.195 75.365) (end 180.28 75.28) (width 0.2) (layer "F.Cu") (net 11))
 (segment (start 180.95 72.65) (end 181.0515 72.5485) (width 0.2) (layer "F.Cu") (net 12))
 (segment (start 180.855 77.905) (end 180.95 77.81) (width 0.2) (layer "F.Cu") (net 12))
 (segment (start 178.405 77.905) (end 180.855 77.905) (width 0.2) (layer "F.Cu") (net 12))
 (segment (start 180.95 77.81) (end 180.95 72.65) (width 0.2) (layer "F.Cu") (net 12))
 (segment (start 181.0515 72.5485) (end 185.56 72.5485) (width 0.2) (layer "F.Cu") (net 12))
 (segment (start 157.32125 80.70125) (end 157.29 80.67) (width 0.2) (layer "F.Cu") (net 13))
 (segment (start 157.29 80.67) (end 181.28 80.67) (width 0.2) (layer "F.Cu") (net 13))
 (segment (start 181.8185 75.0885) (end 185.56 75.0885) (width 0.2) (layer "F.Cu") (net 13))
 (segment (start 181.28 80.67) (end 181.76 80.19) (width 0.2) (layer "F.Cu") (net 13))
 (segment (start 157.32125 90.17) (end 157.32125 109.22) (width 0.2) (layer "F.Cu") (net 13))
 (segment (start 157.32125 109.22) (end 157.32125 128.27) (width 0.2) (layer "F.Cu") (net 13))
 (segment (start 181.76 80.19) (end 181.76 75.03) (width 0.2) (layer "F.Cu") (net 13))
 (segment (start 157.32125 90.17) (end 157.32125 80.70125) (width 0.2) (layer "F.Cu") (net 13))
 (segment (start 181.76 75.03) (end 181.8185 75.0885) (width 0.2) (layer "F.Cu") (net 13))
 (segment (start 176.37125 109.22) (end 176.37125 128.27) (width 0.2) (layer "F.Cu") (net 15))
 (segment (start 182.33 77.7) (end 182.4015 77.6285) (width 0.2) (layer "F.Cu") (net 15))
 (segment (start 176.37125 81.27875) (end 176.41 81.24) (width 0.2) (layer "F.Cu") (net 15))
 (segment (start 176.37125 90.17) (end 176.37125 81.27875) (width 0.2) (layer "F.Cu") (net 15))
 (segment (start 182.4015 77.6285) (end 185.56 77.6285) (width 0.2) (layer "F.Cu") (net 15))
 (segment (start 176.41 81.24) (end 182.05 81.24) (width 0.2) (layer "F.Cu") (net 15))
 (segment (start 182.05 81.24) (end 182.33 80.96) (width 0.2) (layer "F.Cu") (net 15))
 (segment (start 182.33 80.96) (end 182.33 77.7) (width 0.2) (layer "F.Cu") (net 15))
 (segment (start 176.37125 90.17) (end 176.37125 109.22) (width 0.2) (layer "B.Cu") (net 15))
 (segment (start 183.73 91.24) (end 183.73 109.01) (width 0.2) (layer "F.Cu") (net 7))
 (segment (start 188.22 91.24) (end 183.73 91.24) (width 0.2) (layer "F.Cu") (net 7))
 (segment (start 195.42125 109.22) (end 195.42125 128.27) (width 0.2) (layer "F.Cu") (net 7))
 (segment (start 183.94 109.22) (end 195.42125 109.22) (width 0.2) (layer "F.Cu") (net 7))
 (segment (start 185.56 80.1685) (end 188.22 82.8285) (width 0.2) (layer "F.Cu") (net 7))
 (segment (start 183.73 109.01) (end 183.94 109.22) (width 0.2) (layer "F.Cu") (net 7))
 (segment (start 188.22 82.8285) (end 188.22 91.24) (width 0.2) (layer "F.Cu") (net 7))
 (segment (start 204.049 98.44) (end 203.98 98.371) (width 0.2) (layer "F.Cu") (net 22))
 (segment (start 203.98 75.09) (end 203.9785 75.0885) (width 0.2) (layer "F.Cu") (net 22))
 (segment (start 203.98 98.371) (end 203.98 75.09) (width 0.2) (layer "F.Cu") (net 22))
 (segment (start 204.019 98.47) (end 204.049 98.44) (width 0.2) (layer "F.Cu") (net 22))
 (segment (start 200.22 98.47) (end 204.019 98.47) (width 0.2) (layer "F.Cu") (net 22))
 (segment (start 203.9785 75.0885) (end 200.8 75.0885) (width 0.2) (layer "F.Cu") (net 22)))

